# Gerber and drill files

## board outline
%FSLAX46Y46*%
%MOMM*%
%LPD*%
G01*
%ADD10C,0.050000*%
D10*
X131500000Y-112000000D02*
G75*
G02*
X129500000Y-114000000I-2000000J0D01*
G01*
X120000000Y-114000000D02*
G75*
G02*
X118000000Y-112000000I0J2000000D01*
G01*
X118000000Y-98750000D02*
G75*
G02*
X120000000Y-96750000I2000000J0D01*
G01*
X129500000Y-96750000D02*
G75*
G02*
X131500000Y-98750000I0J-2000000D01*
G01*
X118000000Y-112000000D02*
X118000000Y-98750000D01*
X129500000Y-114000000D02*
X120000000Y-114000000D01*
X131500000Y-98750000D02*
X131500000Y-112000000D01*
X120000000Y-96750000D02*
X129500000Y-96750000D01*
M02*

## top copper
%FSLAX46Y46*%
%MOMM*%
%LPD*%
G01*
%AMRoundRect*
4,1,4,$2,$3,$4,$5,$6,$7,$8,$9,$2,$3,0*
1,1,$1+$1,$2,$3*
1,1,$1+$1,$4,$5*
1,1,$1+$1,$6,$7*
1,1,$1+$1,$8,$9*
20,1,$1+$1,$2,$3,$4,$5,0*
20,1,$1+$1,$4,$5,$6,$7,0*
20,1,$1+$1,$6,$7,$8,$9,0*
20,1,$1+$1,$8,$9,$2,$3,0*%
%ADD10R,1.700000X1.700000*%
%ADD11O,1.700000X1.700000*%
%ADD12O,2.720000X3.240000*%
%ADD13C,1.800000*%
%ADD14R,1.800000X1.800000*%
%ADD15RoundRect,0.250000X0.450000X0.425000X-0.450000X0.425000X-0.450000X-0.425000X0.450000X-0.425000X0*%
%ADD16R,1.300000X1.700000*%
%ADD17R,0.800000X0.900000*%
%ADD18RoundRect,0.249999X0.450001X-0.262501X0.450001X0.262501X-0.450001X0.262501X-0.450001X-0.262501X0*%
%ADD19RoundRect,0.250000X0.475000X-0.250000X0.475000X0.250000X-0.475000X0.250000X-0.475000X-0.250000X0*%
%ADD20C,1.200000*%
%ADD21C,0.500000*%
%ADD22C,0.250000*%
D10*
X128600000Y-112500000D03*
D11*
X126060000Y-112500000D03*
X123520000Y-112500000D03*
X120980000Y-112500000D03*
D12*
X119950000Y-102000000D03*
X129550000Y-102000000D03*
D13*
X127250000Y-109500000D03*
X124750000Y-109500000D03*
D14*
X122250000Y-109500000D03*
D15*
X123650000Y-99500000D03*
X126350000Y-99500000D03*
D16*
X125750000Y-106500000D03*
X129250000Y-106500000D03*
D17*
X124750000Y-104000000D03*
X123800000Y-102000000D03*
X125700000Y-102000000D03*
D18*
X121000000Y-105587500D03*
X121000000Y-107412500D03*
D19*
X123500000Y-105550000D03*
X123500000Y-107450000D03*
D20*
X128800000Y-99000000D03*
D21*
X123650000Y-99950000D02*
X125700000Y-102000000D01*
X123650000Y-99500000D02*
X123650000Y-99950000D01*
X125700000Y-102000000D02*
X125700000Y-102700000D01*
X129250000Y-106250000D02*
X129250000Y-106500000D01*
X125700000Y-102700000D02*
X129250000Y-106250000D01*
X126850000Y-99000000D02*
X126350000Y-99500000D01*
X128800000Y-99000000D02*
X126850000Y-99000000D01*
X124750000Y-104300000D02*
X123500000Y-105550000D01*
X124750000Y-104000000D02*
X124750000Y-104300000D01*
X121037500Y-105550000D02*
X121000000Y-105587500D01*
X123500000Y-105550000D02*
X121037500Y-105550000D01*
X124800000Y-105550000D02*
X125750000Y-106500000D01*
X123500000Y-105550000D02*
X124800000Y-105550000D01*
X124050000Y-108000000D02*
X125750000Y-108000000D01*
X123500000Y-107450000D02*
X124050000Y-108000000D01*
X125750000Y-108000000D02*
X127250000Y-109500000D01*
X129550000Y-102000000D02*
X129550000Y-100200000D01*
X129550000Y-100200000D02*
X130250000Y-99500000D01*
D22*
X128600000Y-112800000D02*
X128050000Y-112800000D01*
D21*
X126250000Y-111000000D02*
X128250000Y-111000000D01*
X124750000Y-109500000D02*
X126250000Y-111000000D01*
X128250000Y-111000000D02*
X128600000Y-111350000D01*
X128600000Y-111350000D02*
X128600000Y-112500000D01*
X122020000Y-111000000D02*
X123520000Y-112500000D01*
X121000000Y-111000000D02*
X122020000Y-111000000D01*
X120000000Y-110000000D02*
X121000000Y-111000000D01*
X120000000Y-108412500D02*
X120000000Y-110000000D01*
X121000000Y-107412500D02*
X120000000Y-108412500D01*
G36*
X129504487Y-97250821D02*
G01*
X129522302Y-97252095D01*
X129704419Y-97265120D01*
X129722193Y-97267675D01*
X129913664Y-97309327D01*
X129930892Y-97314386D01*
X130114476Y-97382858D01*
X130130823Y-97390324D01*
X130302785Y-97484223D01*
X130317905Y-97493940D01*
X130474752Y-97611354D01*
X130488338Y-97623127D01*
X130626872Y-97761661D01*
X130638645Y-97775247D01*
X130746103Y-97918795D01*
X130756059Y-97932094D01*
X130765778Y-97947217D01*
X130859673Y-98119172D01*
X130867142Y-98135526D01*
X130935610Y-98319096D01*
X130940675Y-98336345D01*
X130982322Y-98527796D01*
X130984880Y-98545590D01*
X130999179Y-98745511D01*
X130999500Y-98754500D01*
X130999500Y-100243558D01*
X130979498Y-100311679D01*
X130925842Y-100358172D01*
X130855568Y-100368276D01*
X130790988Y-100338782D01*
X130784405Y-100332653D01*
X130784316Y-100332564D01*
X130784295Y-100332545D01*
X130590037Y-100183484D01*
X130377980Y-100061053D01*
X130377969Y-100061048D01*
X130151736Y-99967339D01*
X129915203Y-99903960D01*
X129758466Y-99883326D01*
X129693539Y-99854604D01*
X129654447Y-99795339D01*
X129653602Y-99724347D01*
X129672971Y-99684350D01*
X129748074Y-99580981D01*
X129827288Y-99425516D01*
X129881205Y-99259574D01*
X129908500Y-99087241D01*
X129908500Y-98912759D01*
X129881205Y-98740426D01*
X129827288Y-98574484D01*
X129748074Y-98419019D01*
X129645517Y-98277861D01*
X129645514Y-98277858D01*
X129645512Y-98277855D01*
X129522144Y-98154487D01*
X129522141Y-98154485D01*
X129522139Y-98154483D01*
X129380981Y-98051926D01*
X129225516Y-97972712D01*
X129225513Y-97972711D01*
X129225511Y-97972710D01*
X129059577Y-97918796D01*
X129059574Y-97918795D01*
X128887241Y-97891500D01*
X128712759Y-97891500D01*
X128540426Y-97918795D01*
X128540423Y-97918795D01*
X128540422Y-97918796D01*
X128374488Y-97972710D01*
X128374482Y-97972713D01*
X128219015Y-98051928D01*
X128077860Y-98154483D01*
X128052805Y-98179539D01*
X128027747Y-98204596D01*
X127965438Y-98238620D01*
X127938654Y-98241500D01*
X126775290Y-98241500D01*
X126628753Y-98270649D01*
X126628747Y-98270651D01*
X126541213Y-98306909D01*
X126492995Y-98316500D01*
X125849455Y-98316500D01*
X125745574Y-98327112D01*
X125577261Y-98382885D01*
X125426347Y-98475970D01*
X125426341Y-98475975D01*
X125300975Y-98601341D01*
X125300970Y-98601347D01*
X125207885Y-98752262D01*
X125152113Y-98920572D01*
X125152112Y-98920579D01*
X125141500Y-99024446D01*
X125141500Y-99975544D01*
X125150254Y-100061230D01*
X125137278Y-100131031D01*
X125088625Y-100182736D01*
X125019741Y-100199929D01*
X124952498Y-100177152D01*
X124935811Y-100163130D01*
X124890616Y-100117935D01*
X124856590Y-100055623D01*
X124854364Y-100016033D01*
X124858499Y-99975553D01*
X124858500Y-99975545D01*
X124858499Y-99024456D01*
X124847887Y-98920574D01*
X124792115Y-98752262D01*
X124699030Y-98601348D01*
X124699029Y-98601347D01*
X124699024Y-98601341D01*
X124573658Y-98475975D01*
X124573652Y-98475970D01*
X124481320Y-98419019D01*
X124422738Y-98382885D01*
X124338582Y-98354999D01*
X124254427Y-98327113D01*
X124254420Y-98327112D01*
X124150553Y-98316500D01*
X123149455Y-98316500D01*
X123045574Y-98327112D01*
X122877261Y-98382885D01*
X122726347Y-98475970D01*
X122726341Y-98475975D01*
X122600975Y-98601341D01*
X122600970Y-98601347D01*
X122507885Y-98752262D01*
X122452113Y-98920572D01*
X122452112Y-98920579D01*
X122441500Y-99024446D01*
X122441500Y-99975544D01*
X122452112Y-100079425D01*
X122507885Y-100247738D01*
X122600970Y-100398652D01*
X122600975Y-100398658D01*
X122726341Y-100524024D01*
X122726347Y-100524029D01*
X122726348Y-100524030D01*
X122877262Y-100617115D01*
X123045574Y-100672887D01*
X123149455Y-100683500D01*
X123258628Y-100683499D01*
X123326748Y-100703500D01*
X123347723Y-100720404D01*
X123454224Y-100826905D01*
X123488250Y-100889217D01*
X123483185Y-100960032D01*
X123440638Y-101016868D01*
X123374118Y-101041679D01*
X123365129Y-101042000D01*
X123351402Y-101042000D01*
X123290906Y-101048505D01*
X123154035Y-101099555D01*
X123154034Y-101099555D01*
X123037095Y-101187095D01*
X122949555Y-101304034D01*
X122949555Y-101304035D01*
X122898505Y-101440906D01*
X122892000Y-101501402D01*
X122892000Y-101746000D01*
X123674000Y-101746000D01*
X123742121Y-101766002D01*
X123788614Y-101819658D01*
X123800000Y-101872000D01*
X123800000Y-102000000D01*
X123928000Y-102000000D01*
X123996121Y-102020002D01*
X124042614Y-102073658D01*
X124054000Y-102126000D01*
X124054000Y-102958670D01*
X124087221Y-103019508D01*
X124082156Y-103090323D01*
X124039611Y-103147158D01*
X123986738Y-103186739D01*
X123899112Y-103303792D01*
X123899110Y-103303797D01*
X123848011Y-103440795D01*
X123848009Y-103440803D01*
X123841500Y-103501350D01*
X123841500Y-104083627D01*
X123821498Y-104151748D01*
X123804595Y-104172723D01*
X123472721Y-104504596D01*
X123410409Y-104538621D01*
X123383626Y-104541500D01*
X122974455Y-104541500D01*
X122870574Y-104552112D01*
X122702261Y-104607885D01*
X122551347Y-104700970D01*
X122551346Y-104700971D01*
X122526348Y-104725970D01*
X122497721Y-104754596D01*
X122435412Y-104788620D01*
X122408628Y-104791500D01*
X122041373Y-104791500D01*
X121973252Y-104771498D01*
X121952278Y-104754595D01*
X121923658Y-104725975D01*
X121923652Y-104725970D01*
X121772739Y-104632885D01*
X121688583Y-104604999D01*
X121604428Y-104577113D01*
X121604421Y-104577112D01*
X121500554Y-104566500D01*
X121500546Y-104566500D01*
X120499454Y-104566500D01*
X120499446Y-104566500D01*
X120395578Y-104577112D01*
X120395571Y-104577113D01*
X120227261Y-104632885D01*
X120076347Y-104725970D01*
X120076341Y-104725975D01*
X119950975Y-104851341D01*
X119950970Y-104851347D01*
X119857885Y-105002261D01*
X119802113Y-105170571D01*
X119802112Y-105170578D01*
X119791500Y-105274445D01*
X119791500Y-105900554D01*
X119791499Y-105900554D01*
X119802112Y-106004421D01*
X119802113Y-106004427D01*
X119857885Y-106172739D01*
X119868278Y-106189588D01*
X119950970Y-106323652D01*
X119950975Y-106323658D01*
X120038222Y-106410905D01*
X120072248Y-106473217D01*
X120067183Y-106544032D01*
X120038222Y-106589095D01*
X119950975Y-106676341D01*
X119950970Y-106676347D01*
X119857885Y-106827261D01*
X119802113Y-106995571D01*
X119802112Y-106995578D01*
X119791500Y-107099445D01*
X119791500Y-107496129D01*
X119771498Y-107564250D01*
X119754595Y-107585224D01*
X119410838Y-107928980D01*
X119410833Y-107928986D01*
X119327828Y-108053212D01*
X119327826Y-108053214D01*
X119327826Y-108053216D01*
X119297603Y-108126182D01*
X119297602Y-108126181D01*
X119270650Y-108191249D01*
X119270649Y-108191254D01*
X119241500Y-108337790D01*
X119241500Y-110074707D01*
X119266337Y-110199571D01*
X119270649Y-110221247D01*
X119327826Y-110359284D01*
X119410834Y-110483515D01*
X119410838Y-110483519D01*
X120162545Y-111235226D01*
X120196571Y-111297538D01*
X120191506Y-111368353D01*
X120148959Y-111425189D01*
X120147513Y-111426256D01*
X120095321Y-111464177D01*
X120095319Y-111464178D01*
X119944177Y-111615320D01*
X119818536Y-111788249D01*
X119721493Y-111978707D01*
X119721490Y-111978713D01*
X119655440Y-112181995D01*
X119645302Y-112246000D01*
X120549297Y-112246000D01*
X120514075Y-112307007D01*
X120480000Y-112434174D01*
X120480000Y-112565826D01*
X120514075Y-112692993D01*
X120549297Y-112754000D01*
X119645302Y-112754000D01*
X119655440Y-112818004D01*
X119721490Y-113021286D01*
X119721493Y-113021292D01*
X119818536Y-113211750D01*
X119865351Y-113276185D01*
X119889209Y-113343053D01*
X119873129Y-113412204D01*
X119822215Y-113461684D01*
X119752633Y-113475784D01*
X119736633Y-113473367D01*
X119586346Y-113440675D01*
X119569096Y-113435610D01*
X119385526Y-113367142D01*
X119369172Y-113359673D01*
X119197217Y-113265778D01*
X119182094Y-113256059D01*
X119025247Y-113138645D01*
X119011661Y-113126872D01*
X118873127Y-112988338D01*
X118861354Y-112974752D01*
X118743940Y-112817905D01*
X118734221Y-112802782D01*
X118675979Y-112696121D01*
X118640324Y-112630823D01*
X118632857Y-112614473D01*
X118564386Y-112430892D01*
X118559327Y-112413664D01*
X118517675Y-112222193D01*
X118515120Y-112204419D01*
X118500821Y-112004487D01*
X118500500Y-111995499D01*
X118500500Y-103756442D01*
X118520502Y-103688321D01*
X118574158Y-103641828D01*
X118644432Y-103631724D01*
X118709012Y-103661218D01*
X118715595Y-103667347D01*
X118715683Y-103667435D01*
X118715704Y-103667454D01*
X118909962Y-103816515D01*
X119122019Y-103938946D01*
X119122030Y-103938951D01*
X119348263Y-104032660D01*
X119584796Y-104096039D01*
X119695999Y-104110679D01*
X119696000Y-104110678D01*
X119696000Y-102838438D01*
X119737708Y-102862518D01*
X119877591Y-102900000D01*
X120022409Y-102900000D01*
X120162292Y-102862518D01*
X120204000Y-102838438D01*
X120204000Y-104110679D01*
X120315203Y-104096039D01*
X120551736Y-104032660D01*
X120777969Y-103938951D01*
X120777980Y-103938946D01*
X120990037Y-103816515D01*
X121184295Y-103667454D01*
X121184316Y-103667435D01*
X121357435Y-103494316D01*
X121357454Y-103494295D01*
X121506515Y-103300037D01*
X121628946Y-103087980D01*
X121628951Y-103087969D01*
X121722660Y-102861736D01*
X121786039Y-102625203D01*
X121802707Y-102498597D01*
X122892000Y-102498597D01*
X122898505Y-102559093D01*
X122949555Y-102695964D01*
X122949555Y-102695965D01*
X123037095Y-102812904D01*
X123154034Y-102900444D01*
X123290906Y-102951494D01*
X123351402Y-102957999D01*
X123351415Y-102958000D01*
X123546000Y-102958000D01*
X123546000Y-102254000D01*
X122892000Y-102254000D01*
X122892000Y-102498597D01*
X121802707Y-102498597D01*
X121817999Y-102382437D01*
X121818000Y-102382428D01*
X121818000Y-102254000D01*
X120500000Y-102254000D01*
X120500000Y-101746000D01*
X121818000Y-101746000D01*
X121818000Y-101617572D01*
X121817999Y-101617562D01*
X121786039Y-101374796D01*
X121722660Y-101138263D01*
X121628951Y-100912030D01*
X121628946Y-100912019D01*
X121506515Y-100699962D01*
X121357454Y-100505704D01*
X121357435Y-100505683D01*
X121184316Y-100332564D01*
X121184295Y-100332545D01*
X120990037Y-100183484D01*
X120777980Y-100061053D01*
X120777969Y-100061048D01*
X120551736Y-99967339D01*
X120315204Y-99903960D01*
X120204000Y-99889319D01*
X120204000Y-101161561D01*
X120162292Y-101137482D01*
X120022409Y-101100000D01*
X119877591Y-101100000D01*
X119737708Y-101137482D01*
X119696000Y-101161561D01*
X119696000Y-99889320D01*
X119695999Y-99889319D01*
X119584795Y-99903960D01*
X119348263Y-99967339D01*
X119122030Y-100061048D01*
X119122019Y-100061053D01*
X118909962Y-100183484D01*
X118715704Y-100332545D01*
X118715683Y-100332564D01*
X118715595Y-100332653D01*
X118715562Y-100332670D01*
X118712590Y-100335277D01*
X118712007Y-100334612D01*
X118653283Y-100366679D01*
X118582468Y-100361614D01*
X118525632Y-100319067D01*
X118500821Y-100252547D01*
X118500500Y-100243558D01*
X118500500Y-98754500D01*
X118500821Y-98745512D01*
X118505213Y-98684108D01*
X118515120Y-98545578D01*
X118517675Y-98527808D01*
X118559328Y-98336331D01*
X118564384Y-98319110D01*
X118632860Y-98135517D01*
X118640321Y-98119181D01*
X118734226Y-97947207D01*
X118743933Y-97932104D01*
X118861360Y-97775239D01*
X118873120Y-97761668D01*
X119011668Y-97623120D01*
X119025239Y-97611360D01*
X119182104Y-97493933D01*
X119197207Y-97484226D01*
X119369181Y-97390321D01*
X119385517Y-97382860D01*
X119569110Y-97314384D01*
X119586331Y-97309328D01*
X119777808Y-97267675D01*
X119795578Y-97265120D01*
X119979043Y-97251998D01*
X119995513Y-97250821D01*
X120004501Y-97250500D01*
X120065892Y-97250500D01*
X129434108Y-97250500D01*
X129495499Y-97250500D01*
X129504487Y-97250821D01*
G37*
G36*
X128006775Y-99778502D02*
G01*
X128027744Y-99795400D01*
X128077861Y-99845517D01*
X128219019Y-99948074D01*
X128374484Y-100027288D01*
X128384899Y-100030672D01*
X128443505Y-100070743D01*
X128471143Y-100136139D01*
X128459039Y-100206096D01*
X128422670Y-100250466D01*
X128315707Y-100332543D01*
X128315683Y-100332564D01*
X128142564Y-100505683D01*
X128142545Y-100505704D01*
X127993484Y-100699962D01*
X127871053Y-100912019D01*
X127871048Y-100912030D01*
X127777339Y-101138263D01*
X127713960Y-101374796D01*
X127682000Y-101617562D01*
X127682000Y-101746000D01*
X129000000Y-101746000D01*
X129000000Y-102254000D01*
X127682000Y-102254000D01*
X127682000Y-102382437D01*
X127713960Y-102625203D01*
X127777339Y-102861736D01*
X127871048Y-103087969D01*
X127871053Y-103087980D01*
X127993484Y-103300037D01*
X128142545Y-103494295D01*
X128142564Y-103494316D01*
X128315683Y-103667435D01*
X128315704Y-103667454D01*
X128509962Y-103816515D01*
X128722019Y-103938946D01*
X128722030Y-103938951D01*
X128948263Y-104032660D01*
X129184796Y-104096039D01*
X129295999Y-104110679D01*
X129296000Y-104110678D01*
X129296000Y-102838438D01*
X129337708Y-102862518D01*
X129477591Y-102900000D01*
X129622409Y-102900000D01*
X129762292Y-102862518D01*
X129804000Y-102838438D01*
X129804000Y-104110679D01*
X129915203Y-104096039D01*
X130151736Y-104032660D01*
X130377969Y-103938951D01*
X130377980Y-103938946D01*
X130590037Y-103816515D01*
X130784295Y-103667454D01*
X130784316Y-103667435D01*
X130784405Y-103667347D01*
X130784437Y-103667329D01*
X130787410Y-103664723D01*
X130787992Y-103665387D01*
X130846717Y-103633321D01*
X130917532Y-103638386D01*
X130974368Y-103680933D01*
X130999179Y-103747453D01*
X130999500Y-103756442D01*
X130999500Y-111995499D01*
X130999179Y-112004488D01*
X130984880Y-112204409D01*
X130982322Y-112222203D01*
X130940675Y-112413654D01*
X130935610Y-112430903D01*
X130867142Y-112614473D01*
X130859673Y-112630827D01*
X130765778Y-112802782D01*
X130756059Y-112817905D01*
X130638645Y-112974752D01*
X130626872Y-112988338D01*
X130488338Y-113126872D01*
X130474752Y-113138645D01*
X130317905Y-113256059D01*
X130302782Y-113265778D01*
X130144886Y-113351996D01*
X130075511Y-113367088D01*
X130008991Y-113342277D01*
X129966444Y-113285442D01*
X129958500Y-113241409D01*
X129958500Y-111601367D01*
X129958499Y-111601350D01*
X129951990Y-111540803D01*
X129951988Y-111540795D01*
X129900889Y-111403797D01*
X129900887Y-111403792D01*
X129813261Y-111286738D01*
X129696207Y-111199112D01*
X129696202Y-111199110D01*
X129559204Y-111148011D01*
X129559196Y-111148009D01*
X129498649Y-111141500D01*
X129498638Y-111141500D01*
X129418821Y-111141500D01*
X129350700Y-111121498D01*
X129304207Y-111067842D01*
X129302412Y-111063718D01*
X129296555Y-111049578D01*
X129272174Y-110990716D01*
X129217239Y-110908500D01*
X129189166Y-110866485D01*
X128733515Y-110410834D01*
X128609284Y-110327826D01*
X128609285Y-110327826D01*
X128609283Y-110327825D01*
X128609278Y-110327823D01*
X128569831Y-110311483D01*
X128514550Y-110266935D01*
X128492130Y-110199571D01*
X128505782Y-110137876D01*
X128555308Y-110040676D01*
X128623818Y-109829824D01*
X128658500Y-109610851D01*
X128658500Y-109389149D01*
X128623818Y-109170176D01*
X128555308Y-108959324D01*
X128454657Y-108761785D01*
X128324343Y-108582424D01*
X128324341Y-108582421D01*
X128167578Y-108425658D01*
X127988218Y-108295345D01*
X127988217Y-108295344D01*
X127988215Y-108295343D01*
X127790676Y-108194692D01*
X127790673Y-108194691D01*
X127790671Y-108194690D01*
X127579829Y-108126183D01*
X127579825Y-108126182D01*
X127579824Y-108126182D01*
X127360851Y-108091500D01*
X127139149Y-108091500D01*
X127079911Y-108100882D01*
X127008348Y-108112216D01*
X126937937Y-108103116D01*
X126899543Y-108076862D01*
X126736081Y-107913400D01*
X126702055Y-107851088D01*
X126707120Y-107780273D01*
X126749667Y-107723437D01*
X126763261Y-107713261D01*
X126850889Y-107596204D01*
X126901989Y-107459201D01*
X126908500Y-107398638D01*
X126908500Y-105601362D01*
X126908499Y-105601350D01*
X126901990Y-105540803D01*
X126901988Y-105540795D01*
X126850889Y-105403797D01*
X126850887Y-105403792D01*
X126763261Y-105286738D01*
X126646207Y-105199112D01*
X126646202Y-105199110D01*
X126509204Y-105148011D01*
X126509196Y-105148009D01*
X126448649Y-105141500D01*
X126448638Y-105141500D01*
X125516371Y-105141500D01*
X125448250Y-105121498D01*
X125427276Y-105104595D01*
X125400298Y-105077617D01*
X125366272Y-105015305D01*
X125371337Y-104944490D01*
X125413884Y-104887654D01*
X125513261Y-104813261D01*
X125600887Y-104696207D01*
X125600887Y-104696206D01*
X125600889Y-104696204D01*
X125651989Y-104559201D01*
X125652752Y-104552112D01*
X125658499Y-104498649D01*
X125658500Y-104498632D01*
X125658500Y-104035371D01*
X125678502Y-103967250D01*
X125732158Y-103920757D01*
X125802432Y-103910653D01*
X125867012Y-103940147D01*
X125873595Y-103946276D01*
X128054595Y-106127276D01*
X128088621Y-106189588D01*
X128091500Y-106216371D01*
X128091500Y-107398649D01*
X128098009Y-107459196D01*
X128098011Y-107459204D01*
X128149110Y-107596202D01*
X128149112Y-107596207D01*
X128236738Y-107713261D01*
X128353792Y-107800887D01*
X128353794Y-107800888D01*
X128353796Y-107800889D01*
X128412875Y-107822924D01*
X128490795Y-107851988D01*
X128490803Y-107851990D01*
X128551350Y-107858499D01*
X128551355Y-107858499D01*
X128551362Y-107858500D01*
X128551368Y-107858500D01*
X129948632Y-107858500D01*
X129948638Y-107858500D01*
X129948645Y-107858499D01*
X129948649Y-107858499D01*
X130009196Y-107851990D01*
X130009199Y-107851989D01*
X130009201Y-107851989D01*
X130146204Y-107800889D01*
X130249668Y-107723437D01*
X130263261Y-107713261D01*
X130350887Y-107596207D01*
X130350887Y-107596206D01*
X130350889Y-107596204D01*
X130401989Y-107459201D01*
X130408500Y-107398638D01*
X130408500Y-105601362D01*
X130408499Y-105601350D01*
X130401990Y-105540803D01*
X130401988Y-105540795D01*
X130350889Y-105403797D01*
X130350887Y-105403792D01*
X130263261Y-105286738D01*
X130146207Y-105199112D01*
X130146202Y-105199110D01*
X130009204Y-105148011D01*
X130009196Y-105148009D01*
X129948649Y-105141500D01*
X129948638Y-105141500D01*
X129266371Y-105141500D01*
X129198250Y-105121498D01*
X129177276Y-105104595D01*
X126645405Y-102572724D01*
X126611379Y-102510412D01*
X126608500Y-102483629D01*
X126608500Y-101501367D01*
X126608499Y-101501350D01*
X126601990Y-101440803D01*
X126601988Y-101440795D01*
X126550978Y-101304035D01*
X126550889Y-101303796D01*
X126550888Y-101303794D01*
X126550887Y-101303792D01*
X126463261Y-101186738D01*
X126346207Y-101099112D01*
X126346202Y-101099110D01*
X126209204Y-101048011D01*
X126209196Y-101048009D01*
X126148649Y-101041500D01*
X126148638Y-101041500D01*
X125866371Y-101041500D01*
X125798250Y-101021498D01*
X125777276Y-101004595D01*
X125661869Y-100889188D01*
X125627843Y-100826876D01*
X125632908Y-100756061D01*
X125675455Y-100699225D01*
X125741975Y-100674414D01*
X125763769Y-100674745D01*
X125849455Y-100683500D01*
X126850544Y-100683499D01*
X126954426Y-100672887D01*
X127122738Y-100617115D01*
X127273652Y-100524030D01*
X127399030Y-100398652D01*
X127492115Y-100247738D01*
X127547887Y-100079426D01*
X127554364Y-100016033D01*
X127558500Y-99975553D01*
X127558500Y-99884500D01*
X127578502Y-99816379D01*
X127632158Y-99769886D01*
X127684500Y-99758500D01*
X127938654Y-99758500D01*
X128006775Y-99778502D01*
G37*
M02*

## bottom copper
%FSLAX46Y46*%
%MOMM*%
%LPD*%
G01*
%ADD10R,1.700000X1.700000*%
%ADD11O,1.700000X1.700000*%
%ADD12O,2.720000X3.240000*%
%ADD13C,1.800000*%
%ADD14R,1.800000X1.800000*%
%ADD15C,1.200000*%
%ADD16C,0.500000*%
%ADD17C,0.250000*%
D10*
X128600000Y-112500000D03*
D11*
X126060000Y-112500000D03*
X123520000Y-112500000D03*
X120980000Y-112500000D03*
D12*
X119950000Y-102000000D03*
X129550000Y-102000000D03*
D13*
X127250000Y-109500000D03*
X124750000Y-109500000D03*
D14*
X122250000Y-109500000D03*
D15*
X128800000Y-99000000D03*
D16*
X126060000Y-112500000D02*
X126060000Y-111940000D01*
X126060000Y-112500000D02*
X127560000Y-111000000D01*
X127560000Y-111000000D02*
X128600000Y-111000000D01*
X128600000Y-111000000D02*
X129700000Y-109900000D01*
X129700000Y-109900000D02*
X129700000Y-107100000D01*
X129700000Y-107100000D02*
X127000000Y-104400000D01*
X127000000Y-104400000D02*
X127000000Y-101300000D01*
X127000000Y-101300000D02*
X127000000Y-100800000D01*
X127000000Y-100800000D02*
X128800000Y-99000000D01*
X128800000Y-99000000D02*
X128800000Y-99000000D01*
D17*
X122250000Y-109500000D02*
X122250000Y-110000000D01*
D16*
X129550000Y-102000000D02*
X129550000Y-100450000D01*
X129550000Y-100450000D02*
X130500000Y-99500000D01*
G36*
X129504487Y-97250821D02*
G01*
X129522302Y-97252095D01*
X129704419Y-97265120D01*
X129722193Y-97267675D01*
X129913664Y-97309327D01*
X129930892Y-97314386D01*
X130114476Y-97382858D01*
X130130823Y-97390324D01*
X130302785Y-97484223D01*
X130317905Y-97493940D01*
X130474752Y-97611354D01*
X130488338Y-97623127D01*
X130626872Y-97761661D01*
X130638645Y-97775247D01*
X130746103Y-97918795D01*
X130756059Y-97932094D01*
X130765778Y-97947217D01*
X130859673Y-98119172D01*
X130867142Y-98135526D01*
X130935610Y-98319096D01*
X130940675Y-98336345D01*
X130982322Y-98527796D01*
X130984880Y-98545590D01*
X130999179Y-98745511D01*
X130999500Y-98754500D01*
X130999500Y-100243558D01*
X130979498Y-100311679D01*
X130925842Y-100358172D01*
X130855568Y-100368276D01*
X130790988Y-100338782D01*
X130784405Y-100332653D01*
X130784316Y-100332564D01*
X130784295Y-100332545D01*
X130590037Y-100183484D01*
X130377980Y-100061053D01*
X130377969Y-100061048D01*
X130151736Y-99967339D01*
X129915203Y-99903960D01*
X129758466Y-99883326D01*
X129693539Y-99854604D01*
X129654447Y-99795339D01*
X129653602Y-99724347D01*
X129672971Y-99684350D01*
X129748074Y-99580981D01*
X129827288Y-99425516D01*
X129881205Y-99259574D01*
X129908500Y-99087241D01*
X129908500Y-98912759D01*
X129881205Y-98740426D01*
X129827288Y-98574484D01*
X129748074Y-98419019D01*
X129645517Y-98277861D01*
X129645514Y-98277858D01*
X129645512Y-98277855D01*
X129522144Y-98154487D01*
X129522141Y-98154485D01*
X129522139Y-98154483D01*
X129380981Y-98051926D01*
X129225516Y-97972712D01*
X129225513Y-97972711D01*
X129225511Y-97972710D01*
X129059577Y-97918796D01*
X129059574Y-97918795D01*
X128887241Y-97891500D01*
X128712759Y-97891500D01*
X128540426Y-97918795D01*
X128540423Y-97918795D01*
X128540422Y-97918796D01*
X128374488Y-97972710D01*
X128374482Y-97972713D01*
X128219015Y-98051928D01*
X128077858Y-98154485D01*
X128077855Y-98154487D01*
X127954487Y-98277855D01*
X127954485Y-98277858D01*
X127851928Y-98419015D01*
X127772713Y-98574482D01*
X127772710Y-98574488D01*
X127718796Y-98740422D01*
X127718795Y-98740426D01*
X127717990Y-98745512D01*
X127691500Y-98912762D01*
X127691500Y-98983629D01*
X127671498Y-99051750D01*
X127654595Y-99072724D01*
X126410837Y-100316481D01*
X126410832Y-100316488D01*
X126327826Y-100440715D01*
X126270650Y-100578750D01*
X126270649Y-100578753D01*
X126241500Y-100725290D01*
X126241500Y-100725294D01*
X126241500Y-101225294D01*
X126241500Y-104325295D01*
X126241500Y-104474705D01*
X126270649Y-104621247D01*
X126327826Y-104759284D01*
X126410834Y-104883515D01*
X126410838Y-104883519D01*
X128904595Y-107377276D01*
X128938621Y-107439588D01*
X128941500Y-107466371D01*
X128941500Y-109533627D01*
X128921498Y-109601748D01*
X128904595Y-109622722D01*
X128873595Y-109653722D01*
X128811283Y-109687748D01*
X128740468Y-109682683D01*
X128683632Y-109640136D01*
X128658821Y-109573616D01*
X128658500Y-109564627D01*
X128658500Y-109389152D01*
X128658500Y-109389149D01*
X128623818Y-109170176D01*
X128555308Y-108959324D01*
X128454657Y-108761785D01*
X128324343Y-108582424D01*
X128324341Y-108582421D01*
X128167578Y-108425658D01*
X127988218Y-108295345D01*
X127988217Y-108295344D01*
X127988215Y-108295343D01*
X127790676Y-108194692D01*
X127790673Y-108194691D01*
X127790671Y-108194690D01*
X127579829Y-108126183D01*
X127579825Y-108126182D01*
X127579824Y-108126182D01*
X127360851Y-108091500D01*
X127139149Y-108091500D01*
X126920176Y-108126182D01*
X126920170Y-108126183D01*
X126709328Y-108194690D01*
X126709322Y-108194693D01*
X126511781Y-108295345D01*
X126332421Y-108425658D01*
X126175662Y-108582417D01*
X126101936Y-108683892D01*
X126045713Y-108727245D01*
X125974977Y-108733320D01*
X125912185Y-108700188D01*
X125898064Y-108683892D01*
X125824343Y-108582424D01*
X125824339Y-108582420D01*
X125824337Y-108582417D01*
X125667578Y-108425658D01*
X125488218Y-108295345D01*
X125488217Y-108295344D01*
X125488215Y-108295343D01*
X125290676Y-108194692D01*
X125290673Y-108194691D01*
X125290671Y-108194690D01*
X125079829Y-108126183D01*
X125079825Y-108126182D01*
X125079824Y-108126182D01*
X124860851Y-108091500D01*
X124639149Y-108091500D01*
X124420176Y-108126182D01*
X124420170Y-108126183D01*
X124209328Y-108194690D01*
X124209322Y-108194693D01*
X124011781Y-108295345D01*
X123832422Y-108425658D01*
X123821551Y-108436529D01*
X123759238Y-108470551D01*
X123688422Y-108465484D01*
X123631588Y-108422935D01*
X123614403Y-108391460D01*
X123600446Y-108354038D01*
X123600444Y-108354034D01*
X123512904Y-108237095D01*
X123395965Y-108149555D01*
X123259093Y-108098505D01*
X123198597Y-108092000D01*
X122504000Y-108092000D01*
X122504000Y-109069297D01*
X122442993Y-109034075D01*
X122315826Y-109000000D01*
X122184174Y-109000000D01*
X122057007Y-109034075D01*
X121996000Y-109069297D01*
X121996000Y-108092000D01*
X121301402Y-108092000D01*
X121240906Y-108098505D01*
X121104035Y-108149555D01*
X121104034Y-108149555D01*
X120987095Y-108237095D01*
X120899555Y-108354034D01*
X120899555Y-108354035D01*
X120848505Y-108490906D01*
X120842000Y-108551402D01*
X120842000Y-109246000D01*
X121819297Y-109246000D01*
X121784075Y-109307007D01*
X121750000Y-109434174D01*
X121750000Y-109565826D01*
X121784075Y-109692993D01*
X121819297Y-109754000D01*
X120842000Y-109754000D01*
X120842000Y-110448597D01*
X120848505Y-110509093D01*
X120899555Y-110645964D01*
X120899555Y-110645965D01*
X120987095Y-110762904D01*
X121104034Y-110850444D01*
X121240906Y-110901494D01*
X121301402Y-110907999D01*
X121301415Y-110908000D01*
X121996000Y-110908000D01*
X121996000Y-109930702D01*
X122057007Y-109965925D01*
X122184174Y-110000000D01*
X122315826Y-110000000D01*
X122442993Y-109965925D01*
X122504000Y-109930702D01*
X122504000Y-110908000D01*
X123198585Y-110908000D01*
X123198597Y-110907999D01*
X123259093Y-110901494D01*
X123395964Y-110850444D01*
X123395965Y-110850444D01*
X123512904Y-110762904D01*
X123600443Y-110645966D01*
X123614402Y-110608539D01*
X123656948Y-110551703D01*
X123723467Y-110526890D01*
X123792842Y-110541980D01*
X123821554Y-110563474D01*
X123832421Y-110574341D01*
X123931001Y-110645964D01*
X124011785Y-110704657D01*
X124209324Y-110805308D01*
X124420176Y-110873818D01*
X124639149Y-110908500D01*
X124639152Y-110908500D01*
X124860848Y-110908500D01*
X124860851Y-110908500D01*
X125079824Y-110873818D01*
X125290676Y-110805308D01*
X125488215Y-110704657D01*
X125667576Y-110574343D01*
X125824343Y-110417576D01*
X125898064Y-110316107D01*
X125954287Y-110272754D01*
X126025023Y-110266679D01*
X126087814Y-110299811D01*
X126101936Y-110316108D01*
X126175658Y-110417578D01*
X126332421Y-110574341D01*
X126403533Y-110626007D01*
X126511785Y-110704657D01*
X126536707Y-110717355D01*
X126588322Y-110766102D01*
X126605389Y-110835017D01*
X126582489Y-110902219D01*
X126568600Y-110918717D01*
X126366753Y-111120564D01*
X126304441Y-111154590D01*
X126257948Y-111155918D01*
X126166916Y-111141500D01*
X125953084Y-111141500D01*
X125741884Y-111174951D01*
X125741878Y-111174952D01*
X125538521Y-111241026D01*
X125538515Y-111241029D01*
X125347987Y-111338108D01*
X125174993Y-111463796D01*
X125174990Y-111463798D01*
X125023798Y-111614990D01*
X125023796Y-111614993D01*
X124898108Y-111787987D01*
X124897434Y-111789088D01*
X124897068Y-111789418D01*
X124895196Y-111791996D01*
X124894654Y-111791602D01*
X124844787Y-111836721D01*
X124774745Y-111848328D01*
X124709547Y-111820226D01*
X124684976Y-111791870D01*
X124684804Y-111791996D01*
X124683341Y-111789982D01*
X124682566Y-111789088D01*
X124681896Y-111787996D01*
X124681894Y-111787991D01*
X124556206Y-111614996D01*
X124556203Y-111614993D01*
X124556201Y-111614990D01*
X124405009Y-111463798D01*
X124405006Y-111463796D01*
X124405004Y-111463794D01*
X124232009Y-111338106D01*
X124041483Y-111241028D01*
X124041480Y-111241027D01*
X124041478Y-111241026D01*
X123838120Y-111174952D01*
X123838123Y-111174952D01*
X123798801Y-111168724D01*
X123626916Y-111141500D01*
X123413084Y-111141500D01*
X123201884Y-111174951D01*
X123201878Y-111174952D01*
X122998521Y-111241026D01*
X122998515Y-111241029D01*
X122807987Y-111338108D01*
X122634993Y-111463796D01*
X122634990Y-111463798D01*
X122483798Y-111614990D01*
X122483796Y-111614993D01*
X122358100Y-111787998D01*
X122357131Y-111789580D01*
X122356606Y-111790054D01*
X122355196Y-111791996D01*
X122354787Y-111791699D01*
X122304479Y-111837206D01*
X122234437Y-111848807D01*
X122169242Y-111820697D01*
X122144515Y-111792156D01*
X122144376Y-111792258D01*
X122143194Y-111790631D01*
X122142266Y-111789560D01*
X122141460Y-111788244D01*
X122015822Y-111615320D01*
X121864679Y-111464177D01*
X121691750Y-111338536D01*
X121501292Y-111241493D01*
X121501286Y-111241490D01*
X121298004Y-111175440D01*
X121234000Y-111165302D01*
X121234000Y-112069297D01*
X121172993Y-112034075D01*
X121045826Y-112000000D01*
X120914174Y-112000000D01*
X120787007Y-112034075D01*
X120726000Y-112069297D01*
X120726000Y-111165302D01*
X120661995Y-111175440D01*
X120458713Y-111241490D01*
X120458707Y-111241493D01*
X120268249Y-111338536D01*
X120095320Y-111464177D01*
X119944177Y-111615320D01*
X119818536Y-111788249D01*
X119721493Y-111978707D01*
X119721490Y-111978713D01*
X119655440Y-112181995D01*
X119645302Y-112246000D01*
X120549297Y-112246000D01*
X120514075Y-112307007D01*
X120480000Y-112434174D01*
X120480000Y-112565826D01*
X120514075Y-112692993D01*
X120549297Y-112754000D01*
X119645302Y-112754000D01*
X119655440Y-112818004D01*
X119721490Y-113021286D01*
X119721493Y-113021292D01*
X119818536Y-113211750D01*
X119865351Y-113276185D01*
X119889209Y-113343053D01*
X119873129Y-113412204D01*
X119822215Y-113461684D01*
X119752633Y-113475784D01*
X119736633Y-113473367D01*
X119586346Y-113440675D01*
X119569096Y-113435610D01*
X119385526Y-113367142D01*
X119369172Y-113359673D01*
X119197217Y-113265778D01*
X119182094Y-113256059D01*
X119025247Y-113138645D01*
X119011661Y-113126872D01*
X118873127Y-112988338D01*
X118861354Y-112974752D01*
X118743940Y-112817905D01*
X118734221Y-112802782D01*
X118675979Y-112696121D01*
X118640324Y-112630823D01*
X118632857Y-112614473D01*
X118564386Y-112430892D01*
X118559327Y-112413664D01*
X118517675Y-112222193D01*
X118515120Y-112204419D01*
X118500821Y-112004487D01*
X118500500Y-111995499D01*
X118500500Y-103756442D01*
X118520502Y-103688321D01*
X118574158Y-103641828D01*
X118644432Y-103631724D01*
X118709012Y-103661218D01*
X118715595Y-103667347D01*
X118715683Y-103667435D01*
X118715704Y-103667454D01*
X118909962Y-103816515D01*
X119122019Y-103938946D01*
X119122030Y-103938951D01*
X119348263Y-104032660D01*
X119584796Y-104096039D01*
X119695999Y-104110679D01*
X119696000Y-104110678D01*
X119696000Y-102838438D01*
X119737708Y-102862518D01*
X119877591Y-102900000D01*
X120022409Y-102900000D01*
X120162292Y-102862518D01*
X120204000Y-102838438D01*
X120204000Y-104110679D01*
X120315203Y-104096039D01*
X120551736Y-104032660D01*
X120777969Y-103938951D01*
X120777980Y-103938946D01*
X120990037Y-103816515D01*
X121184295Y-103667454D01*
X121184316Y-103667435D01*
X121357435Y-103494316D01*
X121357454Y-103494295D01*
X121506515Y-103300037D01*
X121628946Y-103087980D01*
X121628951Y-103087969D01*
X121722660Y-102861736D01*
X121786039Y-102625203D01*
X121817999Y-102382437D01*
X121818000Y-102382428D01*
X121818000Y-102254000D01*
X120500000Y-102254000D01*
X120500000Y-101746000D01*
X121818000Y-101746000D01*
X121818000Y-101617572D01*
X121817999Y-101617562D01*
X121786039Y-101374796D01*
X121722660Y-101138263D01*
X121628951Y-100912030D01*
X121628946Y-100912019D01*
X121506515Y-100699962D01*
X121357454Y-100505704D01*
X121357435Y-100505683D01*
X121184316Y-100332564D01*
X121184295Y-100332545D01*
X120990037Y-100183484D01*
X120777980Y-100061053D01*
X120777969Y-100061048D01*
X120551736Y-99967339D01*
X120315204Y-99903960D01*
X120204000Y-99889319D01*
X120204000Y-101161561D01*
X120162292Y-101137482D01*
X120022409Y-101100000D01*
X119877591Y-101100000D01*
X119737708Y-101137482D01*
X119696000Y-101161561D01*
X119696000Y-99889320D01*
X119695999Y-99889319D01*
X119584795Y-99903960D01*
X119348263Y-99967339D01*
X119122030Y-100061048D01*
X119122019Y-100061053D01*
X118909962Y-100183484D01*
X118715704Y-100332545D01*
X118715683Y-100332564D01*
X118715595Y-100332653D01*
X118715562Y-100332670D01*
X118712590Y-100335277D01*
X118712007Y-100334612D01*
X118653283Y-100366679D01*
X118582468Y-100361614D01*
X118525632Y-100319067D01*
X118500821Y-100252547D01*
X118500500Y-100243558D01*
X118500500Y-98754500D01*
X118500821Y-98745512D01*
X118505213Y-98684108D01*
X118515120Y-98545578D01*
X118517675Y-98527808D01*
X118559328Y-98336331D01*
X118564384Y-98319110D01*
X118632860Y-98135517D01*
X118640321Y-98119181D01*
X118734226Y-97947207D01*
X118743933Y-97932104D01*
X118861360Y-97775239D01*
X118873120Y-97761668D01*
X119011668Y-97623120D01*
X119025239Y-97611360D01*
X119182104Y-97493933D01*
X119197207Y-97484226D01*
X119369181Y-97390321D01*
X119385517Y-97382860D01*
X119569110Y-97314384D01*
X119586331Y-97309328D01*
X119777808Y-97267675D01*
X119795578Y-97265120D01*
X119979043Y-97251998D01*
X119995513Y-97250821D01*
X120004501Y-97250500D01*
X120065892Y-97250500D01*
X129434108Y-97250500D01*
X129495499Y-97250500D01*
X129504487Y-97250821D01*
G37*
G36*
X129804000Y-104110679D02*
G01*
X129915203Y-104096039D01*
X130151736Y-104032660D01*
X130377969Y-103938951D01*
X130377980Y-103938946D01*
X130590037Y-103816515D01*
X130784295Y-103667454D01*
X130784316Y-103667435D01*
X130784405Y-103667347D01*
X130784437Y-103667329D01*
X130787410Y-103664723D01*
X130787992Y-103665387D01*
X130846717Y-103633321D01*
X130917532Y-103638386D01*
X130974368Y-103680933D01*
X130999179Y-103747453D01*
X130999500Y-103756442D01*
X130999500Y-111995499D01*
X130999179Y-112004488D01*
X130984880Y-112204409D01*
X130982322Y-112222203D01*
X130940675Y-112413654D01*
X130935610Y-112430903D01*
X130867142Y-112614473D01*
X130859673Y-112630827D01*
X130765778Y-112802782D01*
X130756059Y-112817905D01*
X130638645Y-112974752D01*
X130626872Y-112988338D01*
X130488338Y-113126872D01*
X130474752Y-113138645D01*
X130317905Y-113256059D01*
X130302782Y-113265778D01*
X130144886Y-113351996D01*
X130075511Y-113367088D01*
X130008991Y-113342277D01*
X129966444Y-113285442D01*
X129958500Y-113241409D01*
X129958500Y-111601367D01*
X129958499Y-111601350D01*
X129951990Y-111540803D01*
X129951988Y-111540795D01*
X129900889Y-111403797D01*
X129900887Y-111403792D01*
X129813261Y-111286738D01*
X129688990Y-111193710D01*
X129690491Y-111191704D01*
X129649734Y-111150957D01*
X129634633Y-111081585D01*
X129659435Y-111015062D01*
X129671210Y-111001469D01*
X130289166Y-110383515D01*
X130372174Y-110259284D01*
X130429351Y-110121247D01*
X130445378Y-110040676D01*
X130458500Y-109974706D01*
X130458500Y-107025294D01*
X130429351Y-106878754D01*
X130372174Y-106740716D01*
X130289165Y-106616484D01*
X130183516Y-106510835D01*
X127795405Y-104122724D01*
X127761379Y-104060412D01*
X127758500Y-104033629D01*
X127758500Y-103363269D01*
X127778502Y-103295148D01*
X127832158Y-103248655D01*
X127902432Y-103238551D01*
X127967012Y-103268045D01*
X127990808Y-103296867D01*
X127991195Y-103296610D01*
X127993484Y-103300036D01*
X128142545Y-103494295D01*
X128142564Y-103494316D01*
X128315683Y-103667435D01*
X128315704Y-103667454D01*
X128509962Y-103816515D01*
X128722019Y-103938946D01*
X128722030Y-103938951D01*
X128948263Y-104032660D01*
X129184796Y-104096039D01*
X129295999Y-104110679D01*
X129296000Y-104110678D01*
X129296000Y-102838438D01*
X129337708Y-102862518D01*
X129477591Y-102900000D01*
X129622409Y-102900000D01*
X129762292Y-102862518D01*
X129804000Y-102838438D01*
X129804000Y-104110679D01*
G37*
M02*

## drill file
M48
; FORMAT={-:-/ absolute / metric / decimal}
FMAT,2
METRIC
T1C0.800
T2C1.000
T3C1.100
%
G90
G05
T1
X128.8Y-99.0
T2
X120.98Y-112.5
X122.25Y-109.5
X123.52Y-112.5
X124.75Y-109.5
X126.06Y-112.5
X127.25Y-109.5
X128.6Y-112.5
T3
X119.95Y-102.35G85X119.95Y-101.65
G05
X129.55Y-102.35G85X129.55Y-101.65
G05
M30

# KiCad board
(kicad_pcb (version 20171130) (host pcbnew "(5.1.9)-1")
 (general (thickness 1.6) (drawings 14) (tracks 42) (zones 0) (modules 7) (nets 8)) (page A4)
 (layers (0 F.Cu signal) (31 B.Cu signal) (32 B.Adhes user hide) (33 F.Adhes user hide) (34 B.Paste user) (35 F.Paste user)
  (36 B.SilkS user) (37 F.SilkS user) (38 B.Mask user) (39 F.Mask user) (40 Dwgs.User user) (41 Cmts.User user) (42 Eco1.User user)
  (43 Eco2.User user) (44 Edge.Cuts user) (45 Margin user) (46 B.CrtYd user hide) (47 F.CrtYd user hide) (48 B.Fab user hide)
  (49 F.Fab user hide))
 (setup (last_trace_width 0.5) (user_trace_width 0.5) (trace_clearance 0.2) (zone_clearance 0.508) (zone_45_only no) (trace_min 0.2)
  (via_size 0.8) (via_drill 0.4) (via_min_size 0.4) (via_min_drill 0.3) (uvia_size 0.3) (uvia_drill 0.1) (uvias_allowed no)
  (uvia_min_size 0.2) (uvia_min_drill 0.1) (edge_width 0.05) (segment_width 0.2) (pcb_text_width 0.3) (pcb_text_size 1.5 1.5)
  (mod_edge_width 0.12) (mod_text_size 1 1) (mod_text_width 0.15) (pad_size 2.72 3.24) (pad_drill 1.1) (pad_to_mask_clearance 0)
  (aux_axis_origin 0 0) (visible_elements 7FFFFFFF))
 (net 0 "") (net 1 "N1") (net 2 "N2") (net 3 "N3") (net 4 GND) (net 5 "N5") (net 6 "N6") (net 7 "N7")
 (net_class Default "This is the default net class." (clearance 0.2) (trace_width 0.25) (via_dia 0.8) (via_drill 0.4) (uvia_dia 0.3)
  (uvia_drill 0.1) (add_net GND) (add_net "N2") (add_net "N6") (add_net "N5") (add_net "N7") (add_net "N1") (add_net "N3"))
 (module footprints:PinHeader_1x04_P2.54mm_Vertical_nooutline (layer B.Cu) (at 128.6 112.5 90)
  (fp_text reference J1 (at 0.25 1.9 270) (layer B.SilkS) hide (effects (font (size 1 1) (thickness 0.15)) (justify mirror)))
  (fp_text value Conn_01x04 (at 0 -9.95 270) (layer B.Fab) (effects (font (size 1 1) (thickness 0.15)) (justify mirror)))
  (pad 1 thru_hole rect (at 0 0 90) (size 1.7 1.7) (drill 1) (layers *.Cu *.Mask) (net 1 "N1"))
  (pad 2 thru_hole oval (at 0 -2.54 90) (size 1.7 1.7) (drill 1) (layers *.Cu *.Mask) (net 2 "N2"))
  (pad 3 thru_hole oval (at 0 -5.08 90) (size 1.7 1.7) (drill 1) (layers *.Cu *.Mask) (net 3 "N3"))
  (pad 4 thru_hole oval (at 0 -7.62 90) (size 1.7 1.7) (drill 1) (layers *.Cu *.Mask) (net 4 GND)))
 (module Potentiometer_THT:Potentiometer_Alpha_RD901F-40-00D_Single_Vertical (layer F.Cu) (at 122.25 109.5 90)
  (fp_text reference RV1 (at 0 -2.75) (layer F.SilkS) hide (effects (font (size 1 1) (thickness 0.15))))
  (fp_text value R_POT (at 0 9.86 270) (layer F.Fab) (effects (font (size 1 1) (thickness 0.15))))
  (pad "" thru_hole oval (at 7.5 -2.3 180) (size 2.72 3.24) (drill oval 1.1 1.8) (layers *.Cu *.Mask) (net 4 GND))
  (pad "" thru_hole oval (at 7.5 7.3 180) (size 2.72 3.24) (drill oval 1.1 1.8) (layers *.Cu *.Mask) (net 4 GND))
  (pad 3 thru_hole circle (at 0 5 180) (size 1.8 1.8) (drill 1) (layers *.Cu *.Mask) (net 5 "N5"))
  (pad 2 thru_hole circle (at 0 2.5 180) (size 1.8 1.8) (drill 1) (layers *.Cu *.Mask) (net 1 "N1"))
  (pad 1 thru_hole rect (at 0 0 180) (size 1.8 1.8) (drill 1) (layers *.Cu *.Mask) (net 4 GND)))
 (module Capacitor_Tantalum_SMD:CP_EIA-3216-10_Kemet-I (layer F.Cu) (at 125 99.5 180)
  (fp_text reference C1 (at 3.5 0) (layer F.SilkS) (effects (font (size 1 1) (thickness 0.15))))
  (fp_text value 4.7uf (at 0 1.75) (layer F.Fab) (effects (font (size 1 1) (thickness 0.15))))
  (pad 2 smd roundrect (at 1.35 0 180) (size 1.4 1.35) (layers F.Cu F.Paste F.Mask) (roundrect_rratio 0.185185) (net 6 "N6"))
  (pad 1 smd roundrect (at -1.35 0 180) (size 1.4 1.35) (layers F.Cu F.Paste F.Mask) (roundrect_rratio 0.185185) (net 2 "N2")))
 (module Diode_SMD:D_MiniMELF (layer F.Cu) (at 127.5 106.5 180)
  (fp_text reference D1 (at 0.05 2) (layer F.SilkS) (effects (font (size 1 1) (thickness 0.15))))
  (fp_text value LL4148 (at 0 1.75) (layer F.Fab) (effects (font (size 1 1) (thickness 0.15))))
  (pad 2 smd rect (at 1.75 0 180) (size 1.3 1.7) (layers F.Cu F.Paste F.Mask) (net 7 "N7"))
  (pad 1 smd rect (at -1.75 0 180) (size 1.3 1.7) (layers F.Cu F.Paste F.Mask) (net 6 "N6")))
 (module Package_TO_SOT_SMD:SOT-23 (layer F.Cu) (at 124.75 103 270)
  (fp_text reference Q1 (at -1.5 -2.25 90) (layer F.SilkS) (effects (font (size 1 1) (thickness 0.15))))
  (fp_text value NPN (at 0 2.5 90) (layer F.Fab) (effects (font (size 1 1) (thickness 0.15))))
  (pad 3 smd rect (at 1 0 270) (size 0.9 0.8) (layers F.Cu F.Paste F.Mask) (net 7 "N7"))
  (pad 2 smd rect (at -1 0.95 270) (size 0.9 0.8) (layers F.Cu F.Paste F.Mask) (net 4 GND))
  (pad 1 smd rect (at -1 -0.95 270) (size 0.9 0.8) (layers F.Cu F.Paste F.Mask) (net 6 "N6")))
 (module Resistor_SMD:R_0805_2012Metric (layer F.Cu) (at 121 106.5 90)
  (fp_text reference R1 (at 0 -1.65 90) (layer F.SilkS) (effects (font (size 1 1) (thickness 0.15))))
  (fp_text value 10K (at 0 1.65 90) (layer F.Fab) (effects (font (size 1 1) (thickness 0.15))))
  (pad 2 smd roundrect (at 0.9125 0 90) (size 1.025 1.4) (layers F.Cu F.Paste F.Mask) (roundrect_rratio 0.2439014634146341) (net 7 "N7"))
  (pad 1 smd roundrect (at -0.9125 0 90) (size 1.025 1.4) (layers F.Cu F.Paste F.Mask) (roundrect_rratio 0.2439014634146341) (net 3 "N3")))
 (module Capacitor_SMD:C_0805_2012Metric (layer F.Cu) (at 123.5 106.5 90)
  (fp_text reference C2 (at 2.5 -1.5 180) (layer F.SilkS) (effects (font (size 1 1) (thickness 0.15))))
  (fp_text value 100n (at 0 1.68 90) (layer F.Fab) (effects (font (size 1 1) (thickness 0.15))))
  (pad 2 smd roundrect (at 0.95 0 90) (size 1 1.45) (layers F.Cu F.Paste F.Mask) (roundrect_rratio 0.25) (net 7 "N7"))
  (pad 1 smd roundrect (at -0.95 0 90) (size 1 1.45) (layers F.Cu F.Paste F.Mask) (roundrect_rratio 0.25) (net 5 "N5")))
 (gr_arc (start 129.5 112) (end 129.5 114) (angle -90) (layer Edge.Cuts) (width 0.05))
 (gr_arc (start 120 112) (end 118 112) (angle -90) (layer Edge.Cuts) (width 0.05))
 (gr_arc (start 120 98.75) (end 120 96.75) (angle -90) (layer Edge.Cuts) (width 0.05))
 (gr_arc (start 129.5 98.75) (end 131.5 98.75) (angle -90) (layer Edge.Cuts) (width 0.05))
 (gr_line (start 118 112) (end 118 98.75) (layer Edge.Cuts) (width 0.05))
 (gr_line (start 129.5 114) (end 120 114) (layer Edge.Cuts) (width 0.05))
 (gr_line (start 131.5 98.75) (end 131.5 112) (layer Edge.Cuts) (width 0.05))
 (gr_line (start 120 96.75) (end 129.5 96.75) (layer Edge.Cuts) (width 0.05))
 (segment (start 123.65 99.95) (end 125.7 102) (width 0.5) (layer F.Cu) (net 6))
 (segment (start 123.65 99.5) (end 123.65 99.95) (width 0.5) (layer F.Cu) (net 6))
 (segment (start 125.7 102) (end 125.7 102.7) (width 0.5) (layer F.Cu) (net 6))
 (segment (start 129.25 106.25) (end 129.25 106.5) (width 0.5) (layer F.Cu) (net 6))
 (segment (start 125.7 102.7) (end 129.25 106.25) (width 0.5) (layer F.Cu) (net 6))
 (segment (start 126.06 112.5) (end 126.06 111.94) (width 0.5) (layer B.Cu) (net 2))
 (segment (start 126.06 112.5) (end 127.56 111) (width 0.5) (layer B.Cu) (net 2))
 (segment (start 127.56 111) (end 128.6 111) (width 0.5) (layer B.Cu) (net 2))
 (segment (start 128.6 111) (end 129.7 109.9) (width 0.5) (layer B.Cu) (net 2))
 (segment (start 129.7 109.9) (end 129.7 107.1) (width 0.5) (layer B.Cu) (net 2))
 (segment (start 129.7 107.1) (end 127 104.4) (width 0.5) (layer B.Cu) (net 2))
 (segment (start 127 104.4) (end 127 101.3) (width 0.5) (layer B.Cu) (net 2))
 (segment (start 127 101.3) (end 127 100.8) (width 0.5) (layer B.Cu) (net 2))
 (segment (start 127 100.8) (end 128.8 99) (width 0.5) (layer B.Cu) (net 2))
 (segment (start 128.8 99) (end 128.8 99) (width 0.5) (layer B.Cu) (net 2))
 (via (at 128.8 99) (size 1.2) (drill 0.8) (layers F.Cu B.Cu) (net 2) (status 1000000))
 (segment (start 126.85 99) (end 126.35 99.5) (width 0.5) (layer F.Cu) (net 2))
 (segment (start 128.8 99) (end 126.85 99) (width 0.5) (layer F.Cu) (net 2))
 (segment (start 124.75 104.3) (end 123.5 105.55) (width 0.5) (layer F.Cu) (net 7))
 (segment (start 124.75 104) (end 124.75 104.3) (width 0.5) (layer F.Cu) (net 7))
 (segment (start 121.0375 105.55) (end 121 105.5875) (width 0.5) (layer F.Cu) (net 7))
 (segment (start 123.5 105.55) (end 121.0375 105.55) (width 0.5) (layer F.Cu) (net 7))
 (segment (start 124.8 105.55) (end 125.75 106.5) (width 0.5) (layer F.Cu) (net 7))
 (segment (start 123.5 105.55) (end 124.8 105.55) (width 0.5) (layer F.Cu) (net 7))
 (segment (start 124.05 108) (end 125.75 108) (width 0.5) (layer F.Cu) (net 5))
 (segment (start 123.5 107.45) (end 124.05 108) (width 0.5) (layer F.Cu) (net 5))
 (segment (start 125.75 108) (end 127.25 109.5) (width 0.5) (layer F.Cu) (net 5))
 (segment (start 122.25 109.5) (end 122.25 110) (width 0.25) (layer B.Cu) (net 4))
 (segment (start 129.55 102) (end 129.55 100.45) (width 0.5) (layer B.Cu) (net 4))
 (segment (start 129.55 100.45) (end 130.5 99.5) (width 0.5) (layer B.Cu) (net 4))
 (segment (start 129.55 102) (end 129.55 100.2) (width 0.5) (layer F.Cu) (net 4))
 (segment (start 129.55 100.2) (end 130.25 99.5) (width 0.5) (layer F.Cu) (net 4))
 (segment (start 128.6 112.8) (end 128.05 112.8) (width 0.25) (layer F.Cu) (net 1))
 (segment (start 126.25 111) (end 128.25 111) (width 0.5) (layer F.Cu) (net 1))
 (segment (start 124.75 109.5) (end 126.25 111) (width 0.5) (layer F.Cu) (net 1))
 (segment (start 128.25 111) (end 128.6 111.35) (width 0.5) (layer F.Cu) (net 1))
 (segment (start 128.6 111.35) (end 128.6 112.5) (width 0.5) (layer F.Cu) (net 1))
 (segment (start 122.02 111) (end 123.52 112.5) (width 0.5) (layer F.Cu) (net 3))
 (segment (start 121 111) (end 122.02 111) (width 0.5) (layer F.Cu) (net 3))
 (segment (start 120 110) (end 121 111) (width 0.5) (layer F.Cu) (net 3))
 (segment (start 120 108.4125) (end 120 110) (width 0.5) (layer F.Cu) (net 3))
 (segment (start 121 107.4125) (end 120 108.4125) (width 0.5) (layer F.Cu) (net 3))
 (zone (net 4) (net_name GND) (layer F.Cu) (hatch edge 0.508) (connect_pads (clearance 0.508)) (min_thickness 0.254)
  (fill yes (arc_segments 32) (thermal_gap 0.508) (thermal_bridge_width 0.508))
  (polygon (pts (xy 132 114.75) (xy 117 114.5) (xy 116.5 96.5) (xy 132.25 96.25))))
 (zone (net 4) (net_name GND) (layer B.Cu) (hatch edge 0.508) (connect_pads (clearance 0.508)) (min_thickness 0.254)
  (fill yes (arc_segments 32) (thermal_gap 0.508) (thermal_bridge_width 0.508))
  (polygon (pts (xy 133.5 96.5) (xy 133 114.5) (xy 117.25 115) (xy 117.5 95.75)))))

